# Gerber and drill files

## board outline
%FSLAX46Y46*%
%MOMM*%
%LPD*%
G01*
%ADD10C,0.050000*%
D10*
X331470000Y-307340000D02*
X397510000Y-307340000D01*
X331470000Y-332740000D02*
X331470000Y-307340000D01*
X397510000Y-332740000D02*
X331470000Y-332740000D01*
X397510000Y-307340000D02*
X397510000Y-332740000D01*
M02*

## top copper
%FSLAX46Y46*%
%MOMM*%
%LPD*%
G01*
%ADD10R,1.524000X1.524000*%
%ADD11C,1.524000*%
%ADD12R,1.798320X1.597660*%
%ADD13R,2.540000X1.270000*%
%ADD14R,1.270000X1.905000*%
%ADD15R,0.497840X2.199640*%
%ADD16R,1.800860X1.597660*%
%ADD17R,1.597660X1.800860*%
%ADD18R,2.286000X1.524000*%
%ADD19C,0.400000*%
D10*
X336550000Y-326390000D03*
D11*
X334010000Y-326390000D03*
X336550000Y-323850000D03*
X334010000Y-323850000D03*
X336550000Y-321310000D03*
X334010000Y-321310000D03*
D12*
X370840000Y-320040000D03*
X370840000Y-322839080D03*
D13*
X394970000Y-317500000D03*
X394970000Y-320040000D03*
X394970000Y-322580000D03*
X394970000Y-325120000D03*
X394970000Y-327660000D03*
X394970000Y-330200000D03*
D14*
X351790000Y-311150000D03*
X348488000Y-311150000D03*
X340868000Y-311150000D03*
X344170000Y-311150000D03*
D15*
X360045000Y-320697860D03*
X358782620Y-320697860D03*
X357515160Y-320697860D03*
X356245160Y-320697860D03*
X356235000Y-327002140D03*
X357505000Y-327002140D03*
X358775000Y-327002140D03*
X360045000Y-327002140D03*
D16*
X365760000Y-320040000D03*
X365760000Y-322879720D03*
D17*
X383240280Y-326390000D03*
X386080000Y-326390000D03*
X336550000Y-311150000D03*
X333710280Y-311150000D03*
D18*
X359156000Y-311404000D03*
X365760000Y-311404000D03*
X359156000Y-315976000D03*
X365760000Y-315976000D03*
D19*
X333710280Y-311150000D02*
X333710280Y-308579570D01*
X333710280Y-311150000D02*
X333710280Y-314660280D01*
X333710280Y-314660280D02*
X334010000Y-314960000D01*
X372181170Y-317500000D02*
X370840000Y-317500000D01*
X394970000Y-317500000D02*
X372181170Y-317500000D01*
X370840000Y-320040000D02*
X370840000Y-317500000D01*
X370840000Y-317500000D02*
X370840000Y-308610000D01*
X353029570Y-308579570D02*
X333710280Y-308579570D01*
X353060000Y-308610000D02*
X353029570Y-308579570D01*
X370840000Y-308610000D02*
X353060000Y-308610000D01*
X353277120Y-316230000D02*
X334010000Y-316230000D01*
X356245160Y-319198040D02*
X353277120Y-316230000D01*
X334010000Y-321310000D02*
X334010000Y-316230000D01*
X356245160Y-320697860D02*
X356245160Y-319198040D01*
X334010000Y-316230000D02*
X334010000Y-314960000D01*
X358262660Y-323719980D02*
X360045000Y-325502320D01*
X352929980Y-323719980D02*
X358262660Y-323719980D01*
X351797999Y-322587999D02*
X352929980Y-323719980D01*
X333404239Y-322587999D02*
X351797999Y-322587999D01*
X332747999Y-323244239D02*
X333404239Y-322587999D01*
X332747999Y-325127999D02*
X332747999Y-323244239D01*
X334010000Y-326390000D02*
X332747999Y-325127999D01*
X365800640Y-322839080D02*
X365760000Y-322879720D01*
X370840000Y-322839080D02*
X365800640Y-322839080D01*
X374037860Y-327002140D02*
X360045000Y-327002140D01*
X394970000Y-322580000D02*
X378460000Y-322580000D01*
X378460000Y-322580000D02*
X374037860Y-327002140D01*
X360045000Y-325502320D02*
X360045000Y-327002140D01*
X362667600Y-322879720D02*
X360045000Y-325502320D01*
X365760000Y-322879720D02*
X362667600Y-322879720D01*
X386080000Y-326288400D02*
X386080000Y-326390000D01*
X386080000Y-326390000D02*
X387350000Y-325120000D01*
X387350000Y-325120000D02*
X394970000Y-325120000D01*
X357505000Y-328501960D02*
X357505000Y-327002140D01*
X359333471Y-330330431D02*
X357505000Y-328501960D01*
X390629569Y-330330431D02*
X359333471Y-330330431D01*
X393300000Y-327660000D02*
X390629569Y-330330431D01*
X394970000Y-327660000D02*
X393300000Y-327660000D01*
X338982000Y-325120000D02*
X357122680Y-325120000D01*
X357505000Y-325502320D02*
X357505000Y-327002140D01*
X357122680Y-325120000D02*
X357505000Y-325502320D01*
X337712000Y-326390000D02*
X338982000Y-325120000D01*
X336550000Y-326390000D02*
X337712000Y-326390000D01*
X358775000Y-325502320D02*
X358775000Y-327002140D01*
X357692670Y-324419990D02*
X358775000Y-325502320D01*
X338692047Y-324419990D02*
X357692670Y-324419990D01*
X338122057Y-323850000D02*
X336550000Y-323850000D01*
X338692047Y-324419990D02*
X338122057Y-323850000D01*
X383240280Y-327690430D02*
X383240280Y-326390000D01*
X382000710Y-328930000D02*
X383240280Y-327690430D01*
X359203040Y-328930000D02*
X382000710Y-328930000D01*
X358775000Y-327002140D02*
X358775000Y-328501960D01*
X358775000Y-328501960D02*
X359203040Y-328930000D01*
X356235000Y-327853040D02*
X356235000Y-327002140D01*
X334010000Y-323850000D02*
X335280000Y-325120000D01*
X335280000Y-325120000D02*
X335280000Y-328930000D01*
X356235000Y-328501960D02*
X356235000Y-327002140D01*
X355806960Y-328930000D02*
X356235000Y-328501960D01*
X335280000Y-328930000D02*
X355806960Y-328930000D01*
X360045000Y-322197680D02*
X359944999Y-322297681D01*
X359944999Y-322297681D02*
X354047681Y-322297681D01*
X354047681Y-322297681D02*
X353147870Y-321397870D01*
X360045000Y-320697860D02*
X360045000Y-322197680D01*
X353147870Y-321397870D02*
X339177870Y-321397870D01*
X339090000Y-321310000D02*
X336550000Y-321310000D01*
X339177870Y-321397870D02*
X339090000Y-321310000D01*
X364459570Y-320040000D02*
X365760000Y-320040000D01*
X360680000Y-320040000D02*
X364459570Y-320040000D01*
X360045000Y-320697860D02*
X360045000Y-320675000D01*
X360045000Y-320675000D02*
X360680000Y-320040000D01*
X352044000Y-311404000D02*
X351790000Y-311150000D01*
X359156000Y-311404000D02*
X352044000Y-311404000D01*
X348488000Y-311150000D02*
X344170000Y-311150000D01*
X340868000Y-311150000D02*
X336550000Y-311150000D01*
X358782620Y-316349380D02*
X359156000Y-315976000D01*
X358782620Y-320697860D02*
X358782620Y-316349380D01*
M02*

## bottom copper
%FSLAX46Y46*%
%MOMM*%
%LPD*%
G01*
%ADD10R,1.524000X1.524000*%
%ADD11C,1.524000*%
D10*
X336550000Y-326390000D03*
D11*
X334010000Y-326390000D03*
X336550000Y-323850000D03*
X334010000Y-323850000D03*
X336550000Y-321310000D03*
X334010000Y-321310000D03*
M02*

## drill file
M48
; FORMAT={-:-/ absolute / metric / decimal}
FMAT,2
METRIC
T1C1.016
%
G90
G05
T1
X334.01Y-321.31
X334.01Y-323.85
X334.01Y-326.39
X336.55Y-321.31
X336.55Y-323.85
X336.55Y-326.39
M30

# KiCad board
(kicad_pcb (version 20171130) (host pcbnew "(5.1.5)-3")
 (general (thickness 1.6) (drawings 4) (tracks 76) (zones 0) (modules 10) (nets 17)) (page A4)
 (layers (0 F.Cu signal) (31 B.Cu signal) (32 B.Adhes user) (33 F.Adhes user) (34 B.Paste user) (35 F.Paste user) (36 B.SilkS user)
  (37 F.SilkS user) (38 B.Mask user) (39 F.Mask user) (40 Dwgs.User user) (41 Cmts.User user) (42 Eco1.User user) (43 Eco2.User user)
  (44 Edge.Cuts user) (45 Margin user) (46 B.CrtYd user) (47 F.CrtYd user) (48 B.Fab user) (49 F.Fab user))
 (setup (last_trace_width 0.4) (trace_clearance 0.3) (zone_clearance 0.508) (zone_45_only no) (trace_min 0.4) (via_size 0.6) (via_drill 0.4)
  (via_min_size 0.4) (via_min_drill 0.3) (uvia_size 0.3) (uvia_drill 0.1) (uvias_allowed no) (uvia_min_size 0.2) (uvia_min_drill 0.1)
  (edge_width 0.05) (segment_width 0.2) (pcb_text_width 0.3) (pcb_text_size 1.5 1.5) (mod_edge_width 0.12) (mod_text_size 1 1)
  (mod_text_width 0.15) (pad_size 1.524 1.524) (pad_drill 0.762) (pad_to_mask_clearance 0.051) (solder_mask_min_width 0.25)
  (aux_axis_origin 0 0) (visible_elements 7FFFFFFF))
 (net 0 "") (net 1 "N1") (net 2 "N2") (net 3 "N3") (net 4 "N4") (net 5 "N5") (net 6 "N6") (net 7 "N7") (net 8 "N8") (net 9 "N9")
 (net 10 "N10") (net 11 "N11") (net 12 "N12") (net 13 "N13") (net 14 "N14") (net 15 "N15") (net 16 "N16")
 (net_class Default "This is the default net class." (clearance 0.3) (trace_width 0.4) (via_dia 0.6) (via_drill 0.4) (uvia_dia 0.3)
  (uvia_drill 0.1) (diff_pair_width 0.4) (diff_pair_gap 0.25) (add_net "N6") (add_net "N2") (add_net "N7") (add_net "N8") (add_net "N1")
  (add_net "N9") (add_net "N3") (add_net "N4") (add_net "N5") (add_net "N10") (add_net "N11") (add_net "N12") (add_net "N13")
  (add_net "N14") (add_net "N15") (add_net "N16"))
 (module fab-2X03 (layer F.Cu) (at 335.28 323.85 90)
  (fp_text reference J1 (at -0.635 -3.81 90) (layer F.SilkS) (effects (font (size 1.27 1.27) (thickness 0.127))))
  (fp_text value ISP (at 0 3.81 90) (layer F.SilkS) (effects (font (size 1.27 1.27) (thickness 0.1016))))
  (pad 1 thru_hole rect (at -2.54 1.27 90) (size 1.524 1.524) (drill 1.016) (layers F&B.Cu F.Paste F.SilkS F.Mask) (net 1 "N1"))
  (pad 2 thru_hole circle (at -2.54 -1.27 90) (size 1.524 3.048) (drill 1.016) (layers F&B.Cu F.Paste F.SilkS F.Mask) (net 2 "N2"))
  (pad 3 thru_hole circle (at 0 1.27 90) (size 1.524 3.048) (drill 1.016) (layers F&B.Cu F.Paste F.SilkS F.Mask) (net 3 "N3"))
  (pad 4 thru_hole circle (at 0 -1.27 90) (size 1.524 3.048) (drill 1.016) (layers F&B.Cu F.Paste F.SilkS F.Mask) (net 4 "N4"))
  (pad 5 thru_hole circle (at 2.54 1.27 90) (size 1.524 3.048) (drill 1.016) (layers F&B.Cu F.Paste F.SilkS F.Mask) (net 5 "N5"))
  (pad 6 thru_hole circle (at 2.54 -1.27 90) (size 1.524 3.048) (drill 1.016) (layers F&B.Cu F.Paste F.SilkS F.Mask) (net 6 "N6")))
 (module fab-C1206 (layer F.Cu) (at 370.84 321.43954 270)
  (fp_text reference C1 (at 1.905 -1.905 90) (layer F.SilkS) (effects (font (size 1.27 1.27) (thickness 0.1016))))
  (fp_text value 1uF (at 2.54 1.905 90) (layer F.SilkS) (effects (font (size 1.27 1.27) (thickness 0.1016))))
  (pad 1 smd rect (at -1.39954 0 270) (size 1.59766 1.79832) (layers F.Cu F.Paste F.Mask) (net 6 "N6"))
  (pad 2 smd rect (at 1.39954 0 270) (size 1.59766 1.79832) (layers F.Cu F.Paste F.Mask) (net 2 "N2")))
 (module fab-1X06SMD (layer F.Cu) (at 394.97 323.85)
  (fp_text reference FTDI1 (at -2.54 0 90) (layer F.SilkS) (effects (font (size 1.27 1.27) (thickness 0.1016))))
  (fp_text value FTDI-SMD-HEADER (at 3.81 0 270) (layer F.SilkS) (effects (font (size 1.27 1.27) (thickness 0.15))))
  (pad 1 smd rect (at 0 -6.35) (size 2.54 1.27) (layers F.Cu F.Paste F.Mask) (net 6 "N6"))
  (pad 2 smd rect (at 0 -3.81) (size 2.54 1.27) (layers F.Cu F.Paste F.Mask) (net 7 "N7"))
  (pad 3 smd rect (at 0 -1.27) (size 2.54 1.27) (layers F.Cu F.Paste F.Mask) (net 2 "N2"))
  (pad 4 smd rect (at 0 1.27) (size 2.54 1.27) (layers F.Cu F.Paste F.Mask) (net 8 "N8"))
  (pad 5 smd rect (at 0 3.81) (size 2.54 1.27) (layers F.Cu F.Paste F.Mask) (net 1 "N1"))
  (pad 6 smd rect (at 0 6.35) (size 2.54 1.27) (layers F.Cu F.Paste F.Mask) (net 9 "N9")))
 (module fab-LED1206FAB (layer F.Cu) (at 350.139 311.15 180)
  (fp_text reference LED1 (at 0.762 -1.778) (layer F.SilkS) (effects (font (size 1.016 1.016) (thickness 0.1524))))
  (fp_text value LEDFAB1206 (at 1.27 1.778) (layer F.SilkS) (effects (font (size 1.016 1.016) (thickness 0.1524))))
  (pad 1 smd rect (at -1.651 0 180) (size 1.27 1.905) (layers F.Cu F.Paste F.Mask) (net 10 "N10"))
  (pad 2 smd rect (at 1.651 0 180) (size 1.27 1.905) (layers F.Cu F.Paste F.Mask) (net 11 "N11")))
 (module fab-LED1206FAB (layer F.Cu) (at 342.519 311.15 180)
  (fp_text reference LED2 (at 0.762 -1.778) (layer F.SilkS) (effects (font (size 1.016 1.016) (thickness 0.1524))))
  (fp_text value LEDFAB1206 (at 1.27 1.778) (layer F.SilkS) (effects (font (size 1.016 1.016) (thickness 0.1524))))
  (pad 2 smd rect (at 1.651 0 180) (size 1.27 1.905) (layers F.Cu F.Paste F.Mask) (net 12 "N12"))
  (pad 1 smd rect (at -1.651 0 180) (size 1.27 1.905) (layers F.Cu F.Paste F.Mask) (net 11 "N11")))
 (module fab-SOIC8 (layer F.Cu) (at 358.14 323.85 180)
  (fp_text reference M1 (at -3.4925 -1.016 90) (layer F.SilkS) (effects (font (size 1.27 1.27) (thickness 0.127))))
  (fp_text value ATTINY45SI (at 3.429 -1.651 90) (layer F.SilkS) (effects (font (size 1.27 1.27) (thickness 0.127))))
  (pad 1 smd rect (at -1.905 3.15214 180) (size 0.49784 2.19964) (layers F.Cu F.Paste F.Mask) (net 5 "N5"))
  (pad 2 smd rect (at -0.64262 3.15214 180) (size 0.49784 2.19964) (layers F.Cu F.Paste F.Mask) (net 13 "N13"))
  (pad 3 smd rect (at 0.62484 3.15214 180) (size 0.49784 2.19964) (layers F.Cu F.Paste F.Mask) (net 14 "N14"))
  (pad 4 smd rect (at 1.89484 3.15214 180) (size 0.49784 2.19964) (layers F.Cu F.Paste F.Mask) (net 6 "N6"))
  (pad 5 smd rect (at 1.905 -3.15214 180) (size 0.49784 2.19964) (layers F.Cu F.Paste F.Mask) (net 4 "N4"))
  (pad 6 smd rect (at 0.635 -3.15214 180) (size 0.49784 2.19964) (layers F.Cu F.Paste F.Mask) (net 1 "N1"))
  (pad 7 smd rect (at -0.635 -3.15214 180) (size 0.49784 2.19964) (layers F.Cu F.Paste F.Mask) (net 3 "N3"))
  (pad 8 smd rect (at -1.905 -3.15214 180) (size 0.49784 2.19964) (layers F.Cu F.Paste F.Mask) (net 2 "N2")))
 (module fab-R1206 (layer F.Cu) (at 365.76 321.45986 270)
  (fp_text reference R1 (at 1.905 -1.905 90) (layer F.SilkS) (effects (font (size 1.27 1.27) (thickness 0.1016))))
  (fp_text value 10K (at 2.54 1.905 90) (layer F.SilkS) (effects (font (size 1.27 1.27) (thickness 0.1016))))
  (pad 1 smd rect (at -1.41986 0 270) (size 1.59766 1.80086) (layers F.Cu F.Paste F.Mask) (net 5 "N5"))
  (pad 2 smd rect (at 1.41986 0 270) (size 1.59766 1.80086) (layers F.Cu F.Paste F.Mask) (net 2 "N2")))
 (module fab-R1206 (layer F.Cu) (at 384.66014 326.39 180)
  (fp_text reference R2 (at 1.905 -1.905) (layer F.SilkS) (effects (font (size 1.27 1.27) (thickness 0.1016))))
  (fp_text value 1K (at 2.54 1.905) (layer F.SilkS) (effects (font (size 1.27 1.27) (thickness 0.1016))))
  (pad 2 smd rect (at 1.41986 0 180) (size 1.59766 1.80086) (layers F.Cu F.Paste F.Mask) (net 3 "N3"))
  (pad 1 smd rect (at -1.41986 0 180) (size 1.59766 1.80086) (layers F.Cu F.Paste F.Mask) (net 8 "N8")))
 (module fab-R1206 (layer F.Cu) (at 335.13014 311.15 180)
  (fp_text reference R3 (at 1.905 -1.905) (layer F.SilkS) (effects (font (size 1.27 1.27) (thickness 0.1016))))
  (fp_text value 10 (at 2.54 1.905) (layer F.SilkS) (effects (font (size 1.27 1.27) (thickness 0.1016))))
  (pad 1 smd rect (at -1.41986 0 180) (size 1.59766 1.80086) (layers F.Cu F.Paste F.Mask) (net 12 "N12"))
  (pad 2 smd rect (at 1.41986 0 180) (size 1.59766 1.80086) (layers F.Cu F.Paste F.Mask) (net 6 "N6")))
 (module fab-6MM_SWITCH (layer F.Cu) (at 362.458 313.69)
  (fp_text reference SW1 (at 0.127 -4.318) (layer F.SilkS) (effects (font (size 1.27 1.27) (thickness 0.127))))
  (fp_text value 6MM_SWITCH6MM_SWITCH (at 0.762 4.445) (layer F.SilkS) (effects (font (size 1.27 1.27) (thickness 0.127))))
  (pad 1 smd rect (at -3.302 -2.286) (size 2.286 1.524) (layers F.Cu F.Paste F.Mask) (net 10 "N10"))
  (pad 2 smd rect (at 3.302 -2.286) (size 2.286 1.524) (layers F.Cu F.Paste F.Mask) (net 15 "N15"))
  (pad 3 smd rect (at -3.302 2.286) (size 2.286 1.524) (layers F.Cu F.Paste F.Mask) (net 13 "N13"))
  (pad 4 smd rect (at 3.302 2.286) (size 2.286 1.524) (layers F.Cu F.Paste F.Mask) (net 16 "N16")))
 (gr_line (start 331.47 307.34) (end 397.51 307.34) (layer Edge.Cuts) (width 0.05))
 (gr_line (start 331.47 332.74) (end 331.47 307.34) (layer Edge.Cuts) (width 0.05))
 (gr_line (start 397.51 332.74) (end 331.47 332.74) (layer Edge.Cuts) (width 0.05))
 (gr_line (start 397.51 307.34) (end 397.51 332.74) (layer Edge.Cuts) (width 0.05))
 (segment (start 333.71028 311.15) (end 333.71028 308.57957) (width 0.4) (layer F.Cu) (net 6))
 (segment (start 333.71028 311.15) (end 333.71028 314.66028) (width 0.4) (layer F.Cu) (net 6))
 (segment (start 333.71028 314.66028) (end 334.01 314.96) (width 0.4) (layer F.Cu) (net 6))
 (segment (start 372.18117 317.5) (end 370.84 317.5) (width 0.4) (layer F.Cu) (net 6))
 (segment (start 394.97 317.5) (end 372.18117 317.5) (width 0.4) (layer F.Cu) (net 6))
 (segment (start 370.84 320.04) (end 370.84 317.5) (width 0.4) (layer F.Cu) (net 6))
 (segment (start 370.84 317.5) (end 370.84 308.61) (width 0.4) (layer F.Cu) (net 6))
 (segment (start 353.02957 308.57957) (end 333.71028 308.57957) (width 0.4) (layer F.Cu) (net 6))
 (segment (start 353.06 308.61) (end 353.02957 308.57957) (width 0.4) (layer F.Cu) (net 6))
 (segment (start 370.84 308.61) (end 353.06 308.61) (width 0.4) (layer F.Cu) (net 6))
 (segment (start 353.27712 316.23) (end 334.01 316.23) (width 0.4) (layer F.Cu) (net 6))
 (segment (start 356.24516 319.19804) (end 353.27712 316.23) (width 0.4) (layer F.Cu) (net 6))
 (segment (start 334.01 321.31) (end 334.01 316.23) (width 0.4) (layer F.Cu) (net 6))
 (segment (start 356.24516 320.69786) (end 356.24516 319.19804) (width 0.4) (layer F.Cu) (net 6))
 (segment (start 334.01 316.23) (end 334.01 314.96) (width 0.4) (layer F.Cu) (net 6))
 (segment (start 358.26266 323.71998) (end 360.045 325.50232) (width 0.4) (layer F.Cu) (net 2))
 (segment (start 352.92998 323.71998) (end 358.26266 323.71998) (width 0.4) (layer F.Cu) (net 2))
 (segment (start 351.797999 322.587999) (end 352.92998 323.71998) (width 0.4) (layer F.Cu) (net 2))
 (segment (start 333.404239 322.587999) (end 351.797999 322.587999) (width 0.4) (layer F.Cu) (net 2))
 (segment (start 332.747999 323.244239) (end 333.404239 322.587999) (width 0.4) (layer F.Cu) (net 2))
 (segment (start 332.747999 325.127999) (end 332.747999 323.244239) (width 0.4) (layer F.Cu) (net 2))
 (segment (start 334.01 326.39) (end 332.747999 325.127999) (width 0.4) (layer F.Cu) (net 2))
 (segment (start 365.80064 322.83908) (end 365.76 322.87972) (width 0.4) (layer F.Cu) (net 2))
 (segment (start 370.84 322.83908) (end 365.80064 322.83908) (width 0.4) (layer F.Cu) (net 2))
 (segment (start 374.03786 327.00214) (end 360.045 327.00214) (width 0.4) (layer F.Cu) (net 2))
 (segment (start 394.97 322.58) (end 378.46 322.58) (width 0.4) (layer F.Cu) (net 2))
 (segment (start 378.46 322.58) (end 374.03786 327.00214) (width 0.4) (layer F.Cu) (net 2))
 (segment (start 360.045 325.50232) (end 360.045 327.00214) (width 0.4) (layer F.Cu) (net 2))
 (segment (start 362.6676 322.87972) (end 360.045 325.50232) (width 0.4) (layer F.Cu) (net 2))
 (segment (start 365.76 322.87972) (end 362.6676 322.87972) (width 0.4) (layer F.Cu) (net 2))
 (segment (start 386.08 326.2884) (end 386.08 326.39) (width 0.4) (layer F.Cu) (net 8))
 (segment (start 386.08 326.39) (end 387.35 325.12) (width 0.4) (layer F.Cu) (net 8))
 (segment (start 387.35 325.12) (end 394.97 325.12) (width 0.4) (layer F.Cu) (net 8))
 (segment (start 357.505 328.50196) (end 357.505 327.00214) (width 0.4) (layer F.Cu) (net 1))
 (segment (start 359.333471 330.330431) (end 357.505 328.50196) (width 0.4) (layer F.Cu) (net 1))
 (segment (start 390.629569 330.330431) (end 359.333471 330.330431) (width 0.4) (layer F.Cu) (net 1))
 (segment (start 393.3 327.66) (end 390.629569 330.330431) (width 0.4) (layer F.Cu) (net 1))
 (segment (start 394.97 327.66) (end 393.3 327.66) (width 0.4) (layer F.Cu) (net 1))
 (segment (start 338.982 325.12) (end 357.12268 325.12) (width 0.4) (layer F.Cu) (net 1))
 (segment (start 357.505 325.50232) (end 357.505 327.00214) (width 0.4) (layer F.Cu) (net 1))
 (segment (start 357.12268 325.12) (end 357.505 325.50232) (width 0.4) (layer F.Cu) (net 1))
 (segment (start 337.712 326.39) (end 338.982 325.12) (width 0.4) (layer F.Cu) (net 1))
 (segment (start 336.55 326.39) (end 337.712 326.39) (width 0.4) (layer F.Cu) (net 1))
 (segment (start 358.775 325.50232) (end 358.775 327.00214) (width 0.4) (layer F.Cu) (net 3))
 (segment (start 357.69267 324.41999) (end 358.775 325.50232) (width 0.4) (layer F.Cu) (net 3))
 (segment (start 338.692047 324.41999) (end 357.69267 324.41999) (width 0.4) (layer F.Cu) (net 3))
 (segment (start 338.122057 323.85) (end 336.55 323.85) (width 0.4) (layer F.Cu) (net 3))
 (segment (start 338.692047 324.41999) (end 338.122057 323.85) (width 0.4) (layer F.Cu) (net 3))
 (segment (start 383.24028 327.69043) (end 383.24028 326.39) (width 0.4) (layer F.Cu) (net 3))
 (segment (start 382.00071 328.93) (end 383.24028 327.69043) (width 0.4) (layer F.Cu) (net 3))
 (segment (start 359.20304 328.93) (end 382.00071 328.93) (width 0.4) (layer F.Cu) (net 3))
 (segment (start 358.775 327.00214) (end 358.775 328.50196) (width 0.4) (layer F.Cu) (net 3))
 (segment (start 358.775 328.50196) (end 359.20304 328.93) (width 0.4) (layer F.Cu) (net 3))
 (segment (start 356.235 327.85304) (end 356.235 327.00214) (width 0.4) (layer F.Cu) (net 4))
 (segment (start 334.01 323.85) (end 335.28 325.12) (width 0.4) (layer F.Cu) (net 4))
 (segment (start 335.28 325.12) (end 335.28 328.93) (width 0.4) (layer F.Cu) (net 4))
 (segment (start 356.235 328.50196) (end 356.235 327.00214) (width 0.4) (layer F.Cu) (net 4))
 (segment (start 355.80696 328.93) (end 356.235 328.50196) (width 0.4) (layer F.Cu) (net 4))
 (segment (start 335.28 328.93) (end 355.80696 328.93) (width 0.4) (layer F.Cu) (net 4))
 (segment (start 360.045 322.19768) (end 359.944999 322.297681) (width 0.4) (layer F.Cu) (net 5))
 (segment (start 359.944999 322.297681) (end 354.047681 322.297681) (width 0.4) (layer F.Cu) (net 5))
 (segment (start 354.047681 322.297681) (end 353.14787 321.39787) (width 0.4) (layer F.Cu) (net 5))
 (segment (start 360.045 320.69786) (end 360.045 322.19768) (width 0.4) (layer F.Cu) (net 5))
 (segment (start 353.14787 321.39787) (end 339.17787 321.39787) (width 0.4) (layer F.Cu) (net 5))
 (segment (start 339.09 321.31) (end 336.55 321.31) (width 0.4) (layer F.Cu) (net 5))
 (segment (start 339.17787 321.39787) (end 339.09 321.31) (width 0.4) (layer F.Cu) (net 5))
 (segment (start 364.45957 320.04) (end 365.76 320.04) (width 0.4) (layer F.Cu) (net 5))
 (segment (start 360.68 320.04) (end 364.45957 320.04) (width 0.4) (layer F.Cu) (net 5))
 (segment (start 360.045 320.69786) (end 360.045 320.675) (width 0.4) (layer F.Cu) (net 5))
 (segment (start 360.045 320.675) (end 360.68 320.04) (width 0.4) (layer F.Cu) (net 5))
 (segment (start 352.044 311.404) (end 351.79 311.15) (width 0.4) (layer F.Cu) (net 10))
 (segment (start 359.156 311.404) (end 352.044 311.404) (width 0.4) (layer F.Cu) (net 10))
 (segment (start 348.488 311.15) (end 344.17 311.15) (width 0.4) (layer F.Cu) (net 11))
 (segment (start 340.868 311.15) (end 336.55 311.15) (width 0.4) (layer F.Cu) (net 12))
 (segment (start 358.78262 316.34938) (end 359.156 315.976) (width 0.4) (layer F.Cu) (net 13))
 (segment (start 358.78262 320.69786) (end 358.78262 316.34938) (width 0.4) (layer F.Cu) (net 13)))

